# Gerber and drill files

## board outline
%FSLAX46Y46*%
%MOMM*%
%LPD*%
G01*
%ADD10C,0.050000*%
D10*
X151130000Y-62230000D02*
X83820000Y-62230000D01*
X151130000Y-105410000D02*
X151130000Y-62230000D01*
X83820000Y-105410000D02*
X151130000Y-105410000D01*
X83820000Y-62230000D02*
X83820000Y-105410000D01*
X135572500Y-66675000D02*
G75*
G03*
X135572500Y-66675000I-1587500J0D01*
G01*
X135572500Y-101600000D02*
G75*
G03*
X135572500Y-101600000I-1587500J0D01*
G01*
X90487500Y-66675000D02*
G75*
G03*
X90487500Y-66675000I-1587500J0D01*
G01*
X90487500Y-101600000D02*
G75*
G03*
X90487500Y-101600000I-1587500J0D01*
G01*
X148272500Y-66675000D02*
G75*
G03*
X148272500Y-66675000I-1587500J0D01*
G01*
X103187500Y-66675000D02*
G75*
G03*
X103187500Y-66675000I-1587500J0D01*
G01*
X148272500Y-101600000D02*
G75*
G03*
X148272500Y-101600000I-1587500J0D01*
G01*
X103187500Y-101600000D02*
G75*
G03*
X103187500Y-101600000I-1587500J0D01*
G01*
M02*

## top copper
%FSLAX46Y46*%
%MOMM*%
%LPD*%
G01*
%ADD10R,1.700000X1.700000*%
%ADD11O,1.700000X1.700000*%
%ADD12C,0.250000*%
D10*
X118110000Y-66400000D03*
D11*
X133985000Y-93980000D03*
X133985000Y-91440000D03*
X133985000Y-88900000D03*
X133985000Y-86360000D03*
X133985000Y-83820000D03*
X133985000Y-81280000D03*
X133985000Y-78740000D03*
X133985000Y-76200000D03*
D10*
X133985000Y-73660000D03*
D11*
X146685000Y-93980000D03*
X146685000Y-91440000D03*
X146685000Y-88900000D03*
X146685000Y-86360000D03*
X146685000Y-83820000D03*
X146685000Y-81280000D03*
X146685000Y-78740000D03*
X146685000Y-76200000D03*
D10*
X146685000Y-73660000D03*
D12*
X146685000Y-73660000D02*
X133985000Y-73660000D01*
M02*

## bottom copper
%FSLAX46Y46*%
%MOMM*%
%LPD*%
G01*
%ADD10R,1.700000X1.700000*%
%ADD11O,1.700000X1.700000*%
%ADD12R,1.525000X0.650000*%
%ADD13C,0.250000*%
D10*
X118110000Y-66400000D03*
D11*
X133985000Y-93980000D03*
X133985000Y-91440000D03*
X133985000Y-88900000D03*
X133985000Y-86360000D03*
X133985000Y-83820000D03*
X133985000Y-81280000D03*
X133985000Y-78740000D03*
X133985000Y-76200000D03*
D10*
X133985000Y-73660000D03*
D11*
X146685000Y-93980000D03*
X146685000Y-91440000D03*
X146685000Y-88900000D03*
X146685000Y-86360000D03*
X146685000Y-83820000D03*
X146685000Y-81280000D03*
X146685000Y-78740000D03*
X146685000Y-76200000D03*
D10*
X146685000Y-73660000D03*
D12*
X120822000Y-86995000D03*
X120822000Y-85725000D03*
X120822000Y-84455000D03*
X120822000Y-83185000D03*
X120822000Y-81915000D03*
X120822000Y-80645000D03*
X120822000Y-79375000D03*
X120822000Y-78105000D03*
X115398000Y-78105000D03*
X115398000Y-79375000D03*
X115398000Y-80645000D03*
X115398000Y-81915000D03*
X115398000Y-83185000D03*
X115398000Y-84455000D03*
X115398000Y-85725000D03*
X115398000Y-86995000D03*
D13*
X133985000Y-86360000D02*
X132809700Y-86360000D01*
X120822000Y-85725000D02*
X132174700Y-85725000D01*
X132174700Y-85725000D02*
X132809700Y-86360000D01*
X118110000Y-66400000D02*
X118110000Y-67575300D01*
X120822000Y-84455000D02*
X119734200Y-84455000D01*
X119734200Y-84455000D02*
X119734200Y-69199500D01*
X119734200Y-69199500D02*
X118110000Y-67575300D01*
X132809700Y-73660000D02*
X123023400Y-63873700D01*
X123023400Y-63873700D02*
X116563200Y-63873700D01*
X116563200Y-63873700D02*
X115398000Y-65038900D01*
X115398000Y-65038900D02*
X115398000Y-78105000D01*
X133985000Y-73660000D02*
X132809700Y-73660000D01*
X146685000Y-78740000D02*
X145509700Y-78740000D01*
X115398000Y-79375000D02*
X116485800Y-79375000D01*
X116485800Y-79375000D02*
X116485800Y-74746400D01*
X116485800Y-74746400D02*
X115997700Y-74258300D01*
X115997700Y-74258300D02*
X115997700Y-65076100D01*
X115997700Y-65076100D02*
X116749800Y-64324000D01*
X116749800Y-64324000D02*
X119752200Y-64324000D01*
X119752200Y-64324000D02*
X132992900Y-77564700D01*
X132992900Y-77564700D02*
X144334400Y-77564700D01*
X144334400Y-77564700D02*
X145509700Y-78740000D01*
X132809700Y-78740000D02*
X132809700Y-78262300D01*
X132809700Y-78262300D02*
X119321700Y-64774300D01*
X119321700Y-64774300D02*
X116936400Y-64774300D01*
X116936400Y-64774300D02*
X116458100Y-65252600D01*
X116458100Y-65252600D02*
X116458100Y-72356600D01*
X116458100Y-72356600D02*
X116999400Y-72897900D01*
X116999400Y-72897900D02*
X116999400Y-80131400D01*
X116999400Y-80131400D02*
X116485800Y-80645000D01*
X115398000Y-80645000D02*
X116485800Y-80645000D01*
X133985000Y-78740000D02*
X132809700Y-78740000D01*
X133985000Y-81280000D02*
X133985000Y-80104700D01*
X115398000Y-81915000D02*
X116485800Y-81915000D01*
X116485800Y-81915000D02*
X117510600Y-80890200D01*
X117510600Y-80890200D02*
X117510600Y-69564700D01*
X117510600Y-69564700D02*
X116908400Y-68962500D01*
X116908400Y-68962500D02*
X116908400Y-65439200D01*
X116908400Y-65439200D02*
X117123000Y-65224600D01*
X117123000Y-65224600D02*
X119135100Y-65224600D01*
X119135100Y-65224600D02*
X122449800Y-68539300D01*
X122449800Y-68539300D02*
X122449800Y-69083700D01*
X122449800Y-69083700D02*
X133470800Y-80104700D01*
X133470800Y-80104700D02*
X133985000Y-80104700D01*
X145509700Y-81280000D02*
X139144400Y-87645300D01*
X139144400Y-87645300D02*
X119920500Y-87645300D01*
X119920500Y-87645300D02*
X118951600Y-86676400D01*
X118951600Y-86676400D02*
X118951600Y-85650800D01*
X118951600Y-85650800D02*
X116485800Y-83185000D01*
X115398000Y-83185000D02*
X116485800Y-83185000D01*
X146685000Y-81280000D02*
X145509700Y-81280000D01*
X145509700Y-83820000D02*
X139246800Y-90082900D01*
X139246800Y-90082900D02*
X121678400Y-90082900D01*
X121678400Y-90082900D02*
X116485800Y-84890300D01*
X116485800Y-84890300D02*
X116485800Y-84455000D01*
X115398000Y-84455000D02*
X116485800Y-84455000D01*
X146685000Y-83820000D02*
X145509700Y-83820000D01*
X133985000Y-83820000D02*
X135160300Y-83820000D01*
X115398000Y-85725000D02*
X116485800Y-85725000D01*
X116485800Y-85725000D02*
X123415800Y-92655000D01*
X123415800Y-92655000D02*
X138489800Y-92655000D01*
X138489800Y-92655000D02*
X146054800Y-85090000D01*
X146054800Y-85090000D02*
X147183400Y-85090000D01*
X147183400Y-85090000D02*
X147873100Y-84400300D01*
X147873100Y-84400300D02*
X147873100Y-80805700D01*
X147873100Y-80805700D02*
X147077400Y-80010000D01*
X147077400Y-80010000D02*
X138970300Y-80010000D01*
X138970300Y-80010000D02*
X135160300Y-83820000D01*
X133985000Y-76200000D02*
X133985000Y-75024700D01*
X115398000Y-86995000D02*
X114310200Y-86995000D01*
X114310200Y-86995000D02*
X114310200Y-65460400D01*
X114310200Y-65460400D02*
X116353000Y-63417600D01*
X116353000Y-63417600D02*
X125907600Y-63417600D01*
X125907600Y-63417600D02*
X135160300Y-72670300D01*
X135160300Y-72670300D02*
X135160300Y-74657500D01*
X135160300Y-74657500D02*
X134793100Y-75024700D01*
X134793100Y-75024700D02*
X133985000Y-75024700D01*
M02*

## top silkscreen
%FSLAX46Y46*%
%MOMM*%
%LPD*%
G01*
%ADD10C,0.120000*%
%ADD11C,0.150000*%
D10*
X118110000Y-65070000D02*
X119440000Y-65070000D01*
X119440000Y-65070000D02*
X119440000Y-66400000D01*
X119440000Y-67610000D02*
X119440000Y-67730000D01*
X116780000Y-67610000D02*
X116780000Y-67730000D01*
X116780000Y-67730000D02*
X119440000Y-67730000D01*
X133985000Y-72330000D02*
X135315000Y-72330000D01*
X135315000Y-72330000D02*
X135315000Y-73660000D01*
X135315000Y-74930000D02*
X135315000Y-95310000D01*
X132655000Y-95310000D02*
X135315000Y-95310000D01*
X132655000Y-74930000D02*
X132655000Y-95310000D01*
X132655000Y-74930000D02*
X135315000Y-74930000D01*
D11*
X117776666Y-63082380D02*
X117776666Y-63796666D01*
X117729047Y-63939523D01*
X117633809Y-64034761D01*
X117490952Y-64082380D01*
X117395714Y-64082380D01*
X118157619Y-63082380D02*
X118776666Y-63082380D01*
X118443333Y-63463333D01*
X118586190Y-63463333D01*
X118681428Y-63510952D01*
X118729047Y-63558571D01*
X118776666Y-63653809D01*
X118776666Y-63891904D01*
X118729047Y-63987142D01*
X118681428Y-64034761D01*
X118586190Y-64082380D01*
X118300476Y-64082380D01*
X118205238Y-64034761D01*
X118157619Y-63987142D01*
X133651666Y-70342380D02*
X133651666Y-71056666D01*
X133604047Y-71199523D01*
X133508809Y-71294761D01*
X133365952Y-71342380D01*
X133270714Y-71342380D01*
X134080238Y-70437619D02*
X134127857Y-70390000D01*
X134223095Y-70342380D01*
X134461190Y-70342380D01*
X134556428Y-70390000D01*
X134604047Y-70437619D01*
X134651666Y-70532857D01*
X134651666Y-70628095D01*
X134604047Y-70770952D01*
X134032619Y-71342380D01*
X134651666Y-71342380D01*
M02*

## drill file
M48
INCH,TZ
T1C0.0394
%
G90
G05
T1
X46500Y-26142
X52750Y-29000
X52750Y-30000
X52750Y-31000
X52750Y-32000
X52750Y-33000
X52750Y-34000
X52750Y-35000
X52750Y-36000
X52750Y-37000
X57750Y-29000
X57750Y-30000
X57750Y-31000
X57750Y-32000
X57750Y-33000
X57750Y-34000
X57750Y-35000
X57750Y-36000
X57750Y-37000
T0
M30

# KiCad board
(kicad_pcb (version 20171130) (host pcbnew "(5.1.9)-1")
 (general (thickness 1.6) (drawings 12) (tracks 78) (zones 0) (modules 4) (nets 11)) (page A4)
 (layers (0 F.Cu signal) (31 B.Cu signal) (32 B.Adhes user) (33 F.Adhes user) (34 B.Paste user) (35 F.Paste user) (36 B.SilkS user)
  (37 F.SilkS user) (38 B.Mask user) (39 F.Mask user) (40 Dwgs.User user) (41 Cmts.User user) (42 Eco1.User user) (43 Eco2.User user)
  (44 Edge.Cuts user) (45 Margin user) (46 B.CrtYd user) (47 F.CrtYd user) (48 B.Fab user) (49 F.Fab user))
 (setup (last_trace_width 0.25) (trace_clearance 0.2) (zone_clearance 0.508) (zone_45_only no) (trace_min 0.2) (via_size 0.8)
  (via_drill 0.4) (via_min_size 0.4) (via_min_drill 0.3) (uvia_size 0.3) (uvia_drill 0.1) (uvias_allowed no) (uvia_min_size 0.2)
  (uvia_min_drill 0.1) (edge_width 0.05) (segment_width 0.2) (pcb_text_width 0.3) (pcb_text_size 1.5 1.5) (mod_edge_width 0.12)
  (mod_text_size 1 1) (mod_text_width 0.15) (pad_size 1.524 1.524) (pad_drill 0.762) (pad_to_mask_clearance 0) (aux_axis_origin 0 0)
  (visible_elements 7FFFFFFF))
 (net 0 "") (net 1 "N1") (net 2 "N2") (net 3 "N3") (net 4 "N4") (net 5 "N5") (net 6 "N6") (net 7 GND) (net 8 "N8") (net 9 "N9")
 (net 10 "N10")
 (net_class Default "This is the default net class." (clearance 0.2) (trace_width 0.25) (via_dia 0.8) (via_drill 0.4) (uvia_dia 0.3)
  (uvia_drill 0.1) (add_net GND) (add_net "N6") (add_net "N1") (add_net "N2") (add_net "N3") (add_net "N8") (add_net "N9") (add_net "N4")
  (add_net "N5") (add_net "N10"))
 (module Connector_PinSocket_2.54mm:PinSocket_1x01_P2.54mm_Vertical (layer F.Cu) (at 118.11 66.4)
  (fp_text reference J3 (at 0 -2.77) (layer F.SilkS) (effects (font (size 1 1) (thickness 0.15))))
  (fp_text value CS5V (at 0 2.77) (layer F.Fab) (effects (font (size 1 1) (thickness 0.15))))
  (fp_line (start 0 -1.33) (end 1.33 -1.33) (layer F.SilkS) (width 0.12))
  (fp_line (start 1.33 -1.33) (end 1.33 0) (layer F.SilkS) (width 0.12))
  (fp_line (start 1.33 1.21) (end 1.33 1.33) (layer F.SilkS) (width 0.12))
  (fp_line (start -1.33 1.21) (end -1.33 1.33) (layer F.SilkS) (width 0.12))
  (fp_line (start -1.33 1.33) (end 1.33 1.33) (layer F.SilkS) (width 0.12))
  (pad 1 thru_hole rect (at 0 0) (size 1.7 1.7) (drill 1) (layers *.Cu *.Mask) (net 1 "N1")))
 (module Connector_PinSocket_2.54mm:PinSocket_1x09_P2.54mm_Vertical (layer F.Cu) (at 133.985 73.66)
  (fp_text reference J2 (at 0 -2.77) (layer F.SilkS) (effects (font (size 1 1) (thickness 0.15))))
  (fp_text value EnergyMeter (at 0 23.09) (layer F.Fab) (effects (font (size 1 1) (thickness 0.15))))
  (fp_line (start 0 -1.33) (end 1.33 -1.33) (layer F.SilkS) (width 0.12))
  (fp_line (start 1.33 -1.33) (end 1.33 0) (layer F.SilkS) (width 0.12))
  (fp_line (start 1.33 1.27) (end 1.33 21.65) (layer F.SilkS) (width 0.12))
  (fp_line (start -1.33 21.65) (end 1.33 21.65) (layer F.SilkS) (width 0.12))
  (fp_line (start -1.33 1.27) (end -1.33 21.65) (layer F.SilkS) (width 0.12))
  (fp_line (start -1.33 1.27) (end 1.33 1.27) (layer F.SilkS) (width 0.12))
  (pad 9 thru_hole oval (at 0 20.32) (size 1.7 1.7) (drill 1) (layers *.Cu *.Mask))
  (pad 8 thru_hole oval (at 0 17.78) (size 1.7 1.7) (drill 1) (layers *.Cu *.Mask))
  (pad 7 thru_hole oval (at 0 15.24) (size 1.7 1.7) (drill 1) (layers *.Cu *.Mask))
  (pad 6 thru_hole oval (at 0 12.7) (size 1.7 1.7) (drill 1) (layers *.Cu *.Mask) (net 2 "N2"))
  (pad 5 thru_hole oval (at 0 10.16) (size 1.7 1.7) (drill 1) (layers *.Cu *.Mask) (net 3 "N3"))
  (pad 4 thru_hole oval (at 0 7.62) (size 1.7 1.7) (drill 1) (layers *.Cu *.Mask) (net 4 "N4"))
  (pad 3 thru_hole oval (at 0 5.08) (size 1.7 1.7) (drill 1) (layers *.Cu *.Mask) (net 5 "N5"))
  (pad 2 thru_hole oval (at 0 2.54) (size 1.7 1.7) (drill 1) (layers *.Cu *.Mask) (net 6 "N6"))
  (pad 1 thru_hole rect (at 0 0) (size 1.7 1.7) (drill 1) (layers *.Cu *.Mask) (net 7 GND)))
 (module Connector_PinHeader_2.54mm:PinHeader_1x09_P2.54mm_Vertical (layer B.Cu) (at 146.685 73.66 180)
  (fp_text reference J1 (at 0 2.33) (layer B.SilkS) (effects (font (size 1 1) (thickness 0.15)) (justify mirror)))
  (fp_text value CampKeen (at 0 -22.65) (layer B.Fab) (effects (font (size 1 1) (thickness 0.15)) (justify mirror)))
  (pad 9 thru_hole oval (at 0 -20.32 180) (size 1.7 1.7) (drill 1) (layers *.Cu *.Mask))
  (pad 8 thru_hole oval (at 0 -17.78 180) (size 1.7 1.7) (drill 1) (layers *.Cu *.Mask))
  (pad 7 thru_hole oval (at 0 -15.24 180) (size 1.7 1.7) (drill 1) (layers *.Cu *.Mask))
  (pad 6 thru_hole oval (at 0 -12.7 180) (size 1.7 1.7) (drill 1) (layers *.Cu *.Mask))
  (pad 5 thru_hole oval (at 0 -10.16 180) (size 1.7 1.7) (drill 1) (layers *.Cu *.Mask) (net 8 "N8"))
  (pad 4 thru_hole oval (at 0 -7.62 180) (size 1.7 1.7) (drill 1) (layers *.Cu *.Mask) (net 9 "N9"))
  (pad 3 thru_hole oval (at 0 -5.08 180) (size 1.7 1.7) (drill 1) (layers *.Cu *.Mask) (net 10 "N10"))
  (pad 2 thru_hole oval (at 0 -2.54 180) (size 1.7 1.7) (drill 1) (layers *.Cu *.Mask))
  (pad 1 thru_hole rect (at 0 0 180) (size 1.7 1.7) (drill 1) (layers *.Cu *.Mask) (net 7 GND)))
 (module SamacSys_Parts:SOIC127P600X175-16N (layer B.Cu) (at 118.11 82.55)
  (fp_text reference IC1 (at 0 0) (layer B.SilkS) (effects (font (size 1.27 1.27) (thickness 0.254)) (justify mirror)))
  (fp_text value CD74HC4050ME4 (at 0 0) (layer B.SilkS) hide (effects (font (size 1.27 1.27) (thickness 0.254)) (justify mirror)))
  (pad 16 smd rect (at 2.712 4.445 270) (size 0.65 1.525) (layers B.Cu B.Paste B.Mask))
  (pad 15 smd rect (at 2.712 3.175 270) (size 0.65 1.525) (layers B.Cu B.Paste B.Mask) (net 2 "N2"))
  (pad 14 smd rect (at 2.712 1.905 270) (size 0.65 1.525) (layers B.Cu B.Paste B.Mask) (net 1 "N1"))
  (pad 13 smd rect (at 2.712 0.635 270) (size 0.65 1.525) (layers B.Cu B.Paste B.Mask))
  (pad 12 smd rect (at 2.712 -0.635 270) (size 0.65 1.525) (layers B.Cu B.Paste B.Mask))
  (pad 11 smd rect (at 2.712 -1.905 270) (size 0.65 1.525) (layers B.Cu B.Paste B.Mask))
  (pad 10 smd rect (at 2.712 -3.175 270) (size 0.65 1.525) (layers B.Cu B.Paste B.Mask))
  (pad 9 smd rect (at 2.712 -4.445 270) (size 0.65 1.525) (layers B.Cu B.Paste B.Mask))
  (pad 8 smd rect (at -2.712 -4.445 270) (size 0.65 1.525) (layers B.Cu B.Paste B.Mask) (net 7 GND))
  (pad 7 smd rect (at -2.712 -3.175 270) (size 0.65 1.525) (layers B.Cu B.Paste B.Mask) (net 10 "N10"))
  (pad 6 smd rect (at -2.712 -1.905 270) (size 0.65 1.525) (layers B.Cu B.Paste B.Mask) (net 5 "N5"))
  (pad 5 smd rect (at -2.712 -0.635 270) (size 0.65 1.525) (layers B.Cu B.Paste B.Mask) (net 4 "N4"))
  (pad 4 smd rect (at -2.712 0.635 270) (size 0.65 1.525) (layers B.Cu B.Paste B.Mask) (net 9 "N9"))
  (pad 3 smd rect (at -2.712 1.905 270) (size 0.65 1.525) (layers B.Cu B.Paste B.Mask) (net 8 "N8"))
  (pad 2 smd rect (at -2.712 3.175 270) (size 0.65 1.525) (layers B.Cu B.Paste B.Mask) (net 3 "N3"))
  (pad 1 smd rect (at -2.712 4.445 270) (size 0.65 1.525) (layers B.Cu B.Paste B.Mask) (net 6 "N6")))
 (gr_line (start 151.13 62.23) (end 83.82 62.23) (layer Edge.Cuts) (width 0.05))
 (gr_line (start 151.13 105.41) (end 151.13 62.23) (layer Edge.Cuts) (width 0.05))
 (gr_line (start 83.82 105.41) (end 151.13 105.41) (layer Edge.Cuts) (width 0.05))
 (gr_line (start 83.82 62.23) (end 83.82 105.41) (layer Edge.Cuts) (width 0.05))
 (gr_circle (center 133.985 66.675) (end 135.5725 66.675) (layer Edge.Cuts) (width 0.05))
 (gr_circle (center 133.985 101.6) (end 135.5725 101.6) (layer Edge.Cuts) (width 0.05))
 (gr_circle (center 88.9 66.675) (end 90.4875 66.675) (layer Edge.Cuts) (width 0.05))
 (gr_circle (center 88.9 101.6) (end 90.4875 101.6) (layer Edge.Cuts) (width 0.05))
 (gr_circle (center 146.685 66.675) (end 148.2725 66.675) (layer Edge.Cuts) (width 0.05))
 (gr_circle (center 101.6 66.675) (end 103.1875 66.675) (layer Edge.Cuts) (width 0.05))
 (gr_circle (center 146.685 101.6) (end 148.2725 101.6) (layer Edge.Cuts) (width 0.05))
 (gr_circle (center 101.6 101.6) (end 103.1875 101.6) (layer Edge.Cuts) (width 0.05))
 (segment (start 133.985 86.36) (end 132.8097 86.36) (width 0.25) (layer B.Cu) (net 2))
 (segment (start 120.822 85.725) (end 132.1747 85.725) (width 0.25) (layer B.Cu) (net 2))
 (segment (start 132.1747 85.725) (end 132.8097 86.36) (width 0.25) (layer B.Cu) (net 2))
 (segment (start 118.11 66.4) (end 118.11 67.5753) (width 0.25) (layer B.Cu) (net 1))
 (segment (start 120.822 84.455) (end 119.7342 84.455) (width 0.25) (layer B.Cu) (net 1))
 (segment (start 119.7342 84.455) (end 119.7342 69.1995) (width 0.25) (layer B.Cu) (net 1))
 (segment (start 119.7342 69.1995) (end 118.11 67.5753) (width 0.25) (layer B.Cu) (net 1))
 (segment (start 132.8097 73.66) (end 123.0234 63.8737) (width 0.25) (layer B.Cu) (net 7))
 (segment (start 123.0234 63.8737) (end 116.5632 63.8737) (width 0.25) (layer B.Cu) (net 7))
 (segment (start 116.5632 63.8737) (end 115.398 65.0389) (width 0.25) (layer B.Cu) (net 7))
 (segment (start 115.398 65.0389) (end 115.398 78.105) (width 0.25) (layer B.Cu) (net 7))
 (segment (start 133.985 73.66) (end 132.8097 73.66) (width 0.25) (layer B.Cu) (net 7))
 (segment (start 146.685 73.66) (end 133.985 73.66) (width 0.25) (layer F.Cu) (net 7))
 (segment (start 146.685 78.74) (end 145.5097 78.74) (width 0.25) (layer B.Cu) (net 10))
 (segment (start 115.398 79.375) (end 116.4858 79.375) (width 0.25) (layer B.Cu) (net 10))
 (segment (start 116.4858 79.375) (end 116.4858 74.7464) (width 0.25) (layer B.Cu) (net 10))
 (segment (start 116.4858 74.7464) (end 115.9977 74.2583) (width 0.25) (layer B.Cu) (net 10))
 (segment (start 115.9977 74.2583) (end 115.9977 65.0761) (width 0.25) (layer B.Cu) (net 10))
 (segment (start 115.9977 65.0761) (end 116.7498 64.324) (width 0.25) (layer B.Cu) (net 10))
 (segment (start 116.7498 64.324) (end 119.7522 64.324) (width 0.25) (layer B.Cu) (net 10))
 (segment (start 119.7522 64.324) (end 132.9929 77.5647) (width 0.25) (layer B.Cu) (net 10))
 (segment (start 132.9929 77.5647) (end 144.3344 77.5647) (width 0.25) (layer B.Cu) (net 10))
 (segment (start 144.3344 77.5647) (end 145.5097 78.74) (width 0.25) (layer B.Cu) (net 10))
 (segment (start 132.8097 78.74) (end 132.8097 78.2623) (width 0.25) (layer B.Cu) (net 5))
 (segment (start 132.8097 78.2623) (end 119.3217 64.7743) (width 0.25) (layer B.Cu) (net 5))
 (segment (start 119.3217 64.7743) (end 116.9364 64.7743) (width 0.25) (layer B.Cu) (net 5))
 (segment (start 116.9364 64.7743) (end 116.4581 65.2526) (width 0.25) (layer B.Cu) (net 5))
 (segment (start 116.4581 65.2526) (end 116.4581 72.3566) (width 0.25) (layer B.Cu) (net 5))
 (segment (start 116.4581 72.3566) (end 116.9994 72.8979) (width 0.25) (layer B.Cu) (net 5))
 (segment (start 116.9994 72.8979) (end 116.9994 80.1314) (width 0.25) (layer B.Cu) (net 5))
 (segment (start 116.9994 80.1314) (end 116.4858 80.645) (width 0.25) (layer B.Cu) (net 5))
 (segment (start 115.398 80.645) (end 116.4858 80.645) (width 0.25) (layer B.Cu) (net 5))
 (segment (start 133.985 78.74) (end 132.8097 78.74) (width 0.25) (layer B.Cu) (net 5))
 (segment (start 133.985 81.28) (end 133.985 80.1047) (width 0.25) (layer B.Cu) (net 4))
 (segment (start 115.398 81.915) (end 116.4858 81.915) (width 0.25) (layer B.Cu) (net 4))
 (segment (start 116.4858 81.915) (end 117.5106 80.8902) (width 0.25) (layer B.Cu) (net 4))
 (segment (start 117.5106 80.8902) (end 117.5106 69.5647) (width 0.25) (layer B.Cu) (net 4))
 (segment (start 117.5106 69.5647) (end 116.9084 68.9625) (width 0.25) (layer B.Cu) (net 4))
 (segment (start 116.9084 68.9625) (end 116.9084 65.4392) (width 0.25) (layer B.Cu) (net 4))
 (segment (start 116.9084 65.4392) (end 117.123 65.2246) (width 0.25) (layer B.Cu) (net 4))
 (segment (start 117.123 65.2246) (end 119.1351 65.2246) (width 0.25) (layer B.Cu) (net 4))
 (segment (start 119.1351 65.2246) (end 122.4498 68.5393) (width 0.25) (layer B.Cu) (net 4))
 (segment (start 122.4498 68.5393) (end 122.4498 69.0837) (width 0.25) (layer B.Cu) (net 4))
 (segment (start 122.4498 69.0837) (end 133.4708 80.1047) (width 0.25) (layer B.Cu) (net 4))
 (segment (start 133.4708 80.1047) (end 133.985 80.1047) (width 0.25) (layer B.Cu) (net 4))
 (segment (start 145.5097 81.28) (end 139.1444 87.6453) (width 0.25) (layer B.Cu) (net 9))
 (segment (start 139.1444 87.6453) (end 119.9205 87.6453) (width 0.25) (layer B.Cu) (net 9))
 (segment (start 119.9205 87.6453) (end 118.9516 86.6764) (width 0.25) (layer B.Cu) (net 9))
 (segment (start 118.9516 86.6764) (end 118.9516 85.6508) (width 0.25) (layer B.Cu) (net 9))
 (segment (start 118.9516 85.6508) (end 116.4858 83.185) (width 0.25) (layer B.Cu) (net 9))
 (segment (start 115.398 83.185) (end 116.4858 83.185) (width 0.25) (layer B.Cu) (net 9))
 (segment (start 146.685 81.28) (end 145.5097 81.28) (width 0.25) (layer B.Cu) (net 9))
 (segment (start 145.5097 83.82) (end 139.2468 90.0829) (width 0.25) (layer B.Cu) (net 8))
 (segment (start 139.2468 90.0829) (end 121.6784 90.0829) (width 0.25) (layer B.Cu) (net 8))
 (segment (start 121.6784 90.0829) (end 116.4858 84.8903) (width 0.25) (layer B.Cu) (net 8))
 (segment (start 116.4858 84.8903) (end 116.4858 84.455) (width 0.25) (layer B.Cu) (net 8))
 (segment (start 115.398 84.455) (end 116.4858 84.455) (width 0.25) (layer B.Cu) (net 8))
 (segment (start 146.685 83.82) (end 145.5097 83.82) (width 0.25) (layer B.Cu) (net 8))
 (segment (start 133.985 83.82) (end 135.1603 83.82) (width 0.25) (layer B.Cu) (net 3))
 (segment (start 115.398 85.725) (end 116.4858 85.725) (width 0.25) (layer B.Cu) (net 3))
 (segment (start 116.4858 85.725) (end 123.4158 92.655) (width 0.25) (layer B.Cu) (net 3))
 (segment (start 123.4158 92.655) (end 138.4898 92.655) (width 0.25) (layer B.Cu) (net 3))
 (segment (start 138.4898 92.655) (end 146.0548 85.09) (width 0.25) (layer B.Cu) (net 3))
 (segment (start 146.0548 85.09) (end 147.1834 85.09) (width 0.25) (layer B.Cu) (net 3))
 (segment (start 147.1834 85.09) (end 147.8731 84.4003) (width 0.25) (layer B.Cu) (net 3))
 (segment (start 147.8731 84.4003) (end 147.8731 80.8057) (width 0.25) (layer B.Cu) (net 3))
 (segment (start 147.8731 80.8057) (end 147.0774 80.01) (width 0.25) (layer B.Cu) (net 3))
 (segment (start 147.0774 80.01) (end 138.9703 80.01) (width 0.25) (layer B.Cu) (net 3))
 (segment (start 138.9703 80.01) (end 135.1603 83.82) (width 0.25) (layer B.Cu) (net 3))
 (segment (start 133.985 76.2) (end 133.985 75.0247) (width 0.25) (layer B.Cu) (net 6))
 (segment (start 115.398 86.995) (end 114.3102 86.995) (width 0.25) (layer B.Cu) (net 6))
 (segment (start 114.3102 86.995) (end 114.3102 65.4604) (width 0.25) (layer B.Cu) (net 6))
 (segment (start 114.3102 65.4604) (end 116.353 63.4176) (width 0.25) (layer B.Cu) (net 6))
 (segment (start 116.353 63.4176) (end 125.9076 63.4176) (width 0.25) (layer B.Cu) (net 6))
 (segment (start 125.9076 63.4176) (end 135.1603 72.6703) (width 0.25) (layer B.Cu) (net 6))
 (segment (start 135.1603 72.6703) (end 135.1603 74.6575) (width 0.25) (layer B.Cu) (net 6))
 (segment (start 135.1603 74.6575) (end 134.7931 75.0247) (width 0.25) (layer B.Cu) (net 6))
 (segment (start 134.7931 75.0247) (end 133.985 75.0247) (width 0.25) (layer B.Cu) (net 6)))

